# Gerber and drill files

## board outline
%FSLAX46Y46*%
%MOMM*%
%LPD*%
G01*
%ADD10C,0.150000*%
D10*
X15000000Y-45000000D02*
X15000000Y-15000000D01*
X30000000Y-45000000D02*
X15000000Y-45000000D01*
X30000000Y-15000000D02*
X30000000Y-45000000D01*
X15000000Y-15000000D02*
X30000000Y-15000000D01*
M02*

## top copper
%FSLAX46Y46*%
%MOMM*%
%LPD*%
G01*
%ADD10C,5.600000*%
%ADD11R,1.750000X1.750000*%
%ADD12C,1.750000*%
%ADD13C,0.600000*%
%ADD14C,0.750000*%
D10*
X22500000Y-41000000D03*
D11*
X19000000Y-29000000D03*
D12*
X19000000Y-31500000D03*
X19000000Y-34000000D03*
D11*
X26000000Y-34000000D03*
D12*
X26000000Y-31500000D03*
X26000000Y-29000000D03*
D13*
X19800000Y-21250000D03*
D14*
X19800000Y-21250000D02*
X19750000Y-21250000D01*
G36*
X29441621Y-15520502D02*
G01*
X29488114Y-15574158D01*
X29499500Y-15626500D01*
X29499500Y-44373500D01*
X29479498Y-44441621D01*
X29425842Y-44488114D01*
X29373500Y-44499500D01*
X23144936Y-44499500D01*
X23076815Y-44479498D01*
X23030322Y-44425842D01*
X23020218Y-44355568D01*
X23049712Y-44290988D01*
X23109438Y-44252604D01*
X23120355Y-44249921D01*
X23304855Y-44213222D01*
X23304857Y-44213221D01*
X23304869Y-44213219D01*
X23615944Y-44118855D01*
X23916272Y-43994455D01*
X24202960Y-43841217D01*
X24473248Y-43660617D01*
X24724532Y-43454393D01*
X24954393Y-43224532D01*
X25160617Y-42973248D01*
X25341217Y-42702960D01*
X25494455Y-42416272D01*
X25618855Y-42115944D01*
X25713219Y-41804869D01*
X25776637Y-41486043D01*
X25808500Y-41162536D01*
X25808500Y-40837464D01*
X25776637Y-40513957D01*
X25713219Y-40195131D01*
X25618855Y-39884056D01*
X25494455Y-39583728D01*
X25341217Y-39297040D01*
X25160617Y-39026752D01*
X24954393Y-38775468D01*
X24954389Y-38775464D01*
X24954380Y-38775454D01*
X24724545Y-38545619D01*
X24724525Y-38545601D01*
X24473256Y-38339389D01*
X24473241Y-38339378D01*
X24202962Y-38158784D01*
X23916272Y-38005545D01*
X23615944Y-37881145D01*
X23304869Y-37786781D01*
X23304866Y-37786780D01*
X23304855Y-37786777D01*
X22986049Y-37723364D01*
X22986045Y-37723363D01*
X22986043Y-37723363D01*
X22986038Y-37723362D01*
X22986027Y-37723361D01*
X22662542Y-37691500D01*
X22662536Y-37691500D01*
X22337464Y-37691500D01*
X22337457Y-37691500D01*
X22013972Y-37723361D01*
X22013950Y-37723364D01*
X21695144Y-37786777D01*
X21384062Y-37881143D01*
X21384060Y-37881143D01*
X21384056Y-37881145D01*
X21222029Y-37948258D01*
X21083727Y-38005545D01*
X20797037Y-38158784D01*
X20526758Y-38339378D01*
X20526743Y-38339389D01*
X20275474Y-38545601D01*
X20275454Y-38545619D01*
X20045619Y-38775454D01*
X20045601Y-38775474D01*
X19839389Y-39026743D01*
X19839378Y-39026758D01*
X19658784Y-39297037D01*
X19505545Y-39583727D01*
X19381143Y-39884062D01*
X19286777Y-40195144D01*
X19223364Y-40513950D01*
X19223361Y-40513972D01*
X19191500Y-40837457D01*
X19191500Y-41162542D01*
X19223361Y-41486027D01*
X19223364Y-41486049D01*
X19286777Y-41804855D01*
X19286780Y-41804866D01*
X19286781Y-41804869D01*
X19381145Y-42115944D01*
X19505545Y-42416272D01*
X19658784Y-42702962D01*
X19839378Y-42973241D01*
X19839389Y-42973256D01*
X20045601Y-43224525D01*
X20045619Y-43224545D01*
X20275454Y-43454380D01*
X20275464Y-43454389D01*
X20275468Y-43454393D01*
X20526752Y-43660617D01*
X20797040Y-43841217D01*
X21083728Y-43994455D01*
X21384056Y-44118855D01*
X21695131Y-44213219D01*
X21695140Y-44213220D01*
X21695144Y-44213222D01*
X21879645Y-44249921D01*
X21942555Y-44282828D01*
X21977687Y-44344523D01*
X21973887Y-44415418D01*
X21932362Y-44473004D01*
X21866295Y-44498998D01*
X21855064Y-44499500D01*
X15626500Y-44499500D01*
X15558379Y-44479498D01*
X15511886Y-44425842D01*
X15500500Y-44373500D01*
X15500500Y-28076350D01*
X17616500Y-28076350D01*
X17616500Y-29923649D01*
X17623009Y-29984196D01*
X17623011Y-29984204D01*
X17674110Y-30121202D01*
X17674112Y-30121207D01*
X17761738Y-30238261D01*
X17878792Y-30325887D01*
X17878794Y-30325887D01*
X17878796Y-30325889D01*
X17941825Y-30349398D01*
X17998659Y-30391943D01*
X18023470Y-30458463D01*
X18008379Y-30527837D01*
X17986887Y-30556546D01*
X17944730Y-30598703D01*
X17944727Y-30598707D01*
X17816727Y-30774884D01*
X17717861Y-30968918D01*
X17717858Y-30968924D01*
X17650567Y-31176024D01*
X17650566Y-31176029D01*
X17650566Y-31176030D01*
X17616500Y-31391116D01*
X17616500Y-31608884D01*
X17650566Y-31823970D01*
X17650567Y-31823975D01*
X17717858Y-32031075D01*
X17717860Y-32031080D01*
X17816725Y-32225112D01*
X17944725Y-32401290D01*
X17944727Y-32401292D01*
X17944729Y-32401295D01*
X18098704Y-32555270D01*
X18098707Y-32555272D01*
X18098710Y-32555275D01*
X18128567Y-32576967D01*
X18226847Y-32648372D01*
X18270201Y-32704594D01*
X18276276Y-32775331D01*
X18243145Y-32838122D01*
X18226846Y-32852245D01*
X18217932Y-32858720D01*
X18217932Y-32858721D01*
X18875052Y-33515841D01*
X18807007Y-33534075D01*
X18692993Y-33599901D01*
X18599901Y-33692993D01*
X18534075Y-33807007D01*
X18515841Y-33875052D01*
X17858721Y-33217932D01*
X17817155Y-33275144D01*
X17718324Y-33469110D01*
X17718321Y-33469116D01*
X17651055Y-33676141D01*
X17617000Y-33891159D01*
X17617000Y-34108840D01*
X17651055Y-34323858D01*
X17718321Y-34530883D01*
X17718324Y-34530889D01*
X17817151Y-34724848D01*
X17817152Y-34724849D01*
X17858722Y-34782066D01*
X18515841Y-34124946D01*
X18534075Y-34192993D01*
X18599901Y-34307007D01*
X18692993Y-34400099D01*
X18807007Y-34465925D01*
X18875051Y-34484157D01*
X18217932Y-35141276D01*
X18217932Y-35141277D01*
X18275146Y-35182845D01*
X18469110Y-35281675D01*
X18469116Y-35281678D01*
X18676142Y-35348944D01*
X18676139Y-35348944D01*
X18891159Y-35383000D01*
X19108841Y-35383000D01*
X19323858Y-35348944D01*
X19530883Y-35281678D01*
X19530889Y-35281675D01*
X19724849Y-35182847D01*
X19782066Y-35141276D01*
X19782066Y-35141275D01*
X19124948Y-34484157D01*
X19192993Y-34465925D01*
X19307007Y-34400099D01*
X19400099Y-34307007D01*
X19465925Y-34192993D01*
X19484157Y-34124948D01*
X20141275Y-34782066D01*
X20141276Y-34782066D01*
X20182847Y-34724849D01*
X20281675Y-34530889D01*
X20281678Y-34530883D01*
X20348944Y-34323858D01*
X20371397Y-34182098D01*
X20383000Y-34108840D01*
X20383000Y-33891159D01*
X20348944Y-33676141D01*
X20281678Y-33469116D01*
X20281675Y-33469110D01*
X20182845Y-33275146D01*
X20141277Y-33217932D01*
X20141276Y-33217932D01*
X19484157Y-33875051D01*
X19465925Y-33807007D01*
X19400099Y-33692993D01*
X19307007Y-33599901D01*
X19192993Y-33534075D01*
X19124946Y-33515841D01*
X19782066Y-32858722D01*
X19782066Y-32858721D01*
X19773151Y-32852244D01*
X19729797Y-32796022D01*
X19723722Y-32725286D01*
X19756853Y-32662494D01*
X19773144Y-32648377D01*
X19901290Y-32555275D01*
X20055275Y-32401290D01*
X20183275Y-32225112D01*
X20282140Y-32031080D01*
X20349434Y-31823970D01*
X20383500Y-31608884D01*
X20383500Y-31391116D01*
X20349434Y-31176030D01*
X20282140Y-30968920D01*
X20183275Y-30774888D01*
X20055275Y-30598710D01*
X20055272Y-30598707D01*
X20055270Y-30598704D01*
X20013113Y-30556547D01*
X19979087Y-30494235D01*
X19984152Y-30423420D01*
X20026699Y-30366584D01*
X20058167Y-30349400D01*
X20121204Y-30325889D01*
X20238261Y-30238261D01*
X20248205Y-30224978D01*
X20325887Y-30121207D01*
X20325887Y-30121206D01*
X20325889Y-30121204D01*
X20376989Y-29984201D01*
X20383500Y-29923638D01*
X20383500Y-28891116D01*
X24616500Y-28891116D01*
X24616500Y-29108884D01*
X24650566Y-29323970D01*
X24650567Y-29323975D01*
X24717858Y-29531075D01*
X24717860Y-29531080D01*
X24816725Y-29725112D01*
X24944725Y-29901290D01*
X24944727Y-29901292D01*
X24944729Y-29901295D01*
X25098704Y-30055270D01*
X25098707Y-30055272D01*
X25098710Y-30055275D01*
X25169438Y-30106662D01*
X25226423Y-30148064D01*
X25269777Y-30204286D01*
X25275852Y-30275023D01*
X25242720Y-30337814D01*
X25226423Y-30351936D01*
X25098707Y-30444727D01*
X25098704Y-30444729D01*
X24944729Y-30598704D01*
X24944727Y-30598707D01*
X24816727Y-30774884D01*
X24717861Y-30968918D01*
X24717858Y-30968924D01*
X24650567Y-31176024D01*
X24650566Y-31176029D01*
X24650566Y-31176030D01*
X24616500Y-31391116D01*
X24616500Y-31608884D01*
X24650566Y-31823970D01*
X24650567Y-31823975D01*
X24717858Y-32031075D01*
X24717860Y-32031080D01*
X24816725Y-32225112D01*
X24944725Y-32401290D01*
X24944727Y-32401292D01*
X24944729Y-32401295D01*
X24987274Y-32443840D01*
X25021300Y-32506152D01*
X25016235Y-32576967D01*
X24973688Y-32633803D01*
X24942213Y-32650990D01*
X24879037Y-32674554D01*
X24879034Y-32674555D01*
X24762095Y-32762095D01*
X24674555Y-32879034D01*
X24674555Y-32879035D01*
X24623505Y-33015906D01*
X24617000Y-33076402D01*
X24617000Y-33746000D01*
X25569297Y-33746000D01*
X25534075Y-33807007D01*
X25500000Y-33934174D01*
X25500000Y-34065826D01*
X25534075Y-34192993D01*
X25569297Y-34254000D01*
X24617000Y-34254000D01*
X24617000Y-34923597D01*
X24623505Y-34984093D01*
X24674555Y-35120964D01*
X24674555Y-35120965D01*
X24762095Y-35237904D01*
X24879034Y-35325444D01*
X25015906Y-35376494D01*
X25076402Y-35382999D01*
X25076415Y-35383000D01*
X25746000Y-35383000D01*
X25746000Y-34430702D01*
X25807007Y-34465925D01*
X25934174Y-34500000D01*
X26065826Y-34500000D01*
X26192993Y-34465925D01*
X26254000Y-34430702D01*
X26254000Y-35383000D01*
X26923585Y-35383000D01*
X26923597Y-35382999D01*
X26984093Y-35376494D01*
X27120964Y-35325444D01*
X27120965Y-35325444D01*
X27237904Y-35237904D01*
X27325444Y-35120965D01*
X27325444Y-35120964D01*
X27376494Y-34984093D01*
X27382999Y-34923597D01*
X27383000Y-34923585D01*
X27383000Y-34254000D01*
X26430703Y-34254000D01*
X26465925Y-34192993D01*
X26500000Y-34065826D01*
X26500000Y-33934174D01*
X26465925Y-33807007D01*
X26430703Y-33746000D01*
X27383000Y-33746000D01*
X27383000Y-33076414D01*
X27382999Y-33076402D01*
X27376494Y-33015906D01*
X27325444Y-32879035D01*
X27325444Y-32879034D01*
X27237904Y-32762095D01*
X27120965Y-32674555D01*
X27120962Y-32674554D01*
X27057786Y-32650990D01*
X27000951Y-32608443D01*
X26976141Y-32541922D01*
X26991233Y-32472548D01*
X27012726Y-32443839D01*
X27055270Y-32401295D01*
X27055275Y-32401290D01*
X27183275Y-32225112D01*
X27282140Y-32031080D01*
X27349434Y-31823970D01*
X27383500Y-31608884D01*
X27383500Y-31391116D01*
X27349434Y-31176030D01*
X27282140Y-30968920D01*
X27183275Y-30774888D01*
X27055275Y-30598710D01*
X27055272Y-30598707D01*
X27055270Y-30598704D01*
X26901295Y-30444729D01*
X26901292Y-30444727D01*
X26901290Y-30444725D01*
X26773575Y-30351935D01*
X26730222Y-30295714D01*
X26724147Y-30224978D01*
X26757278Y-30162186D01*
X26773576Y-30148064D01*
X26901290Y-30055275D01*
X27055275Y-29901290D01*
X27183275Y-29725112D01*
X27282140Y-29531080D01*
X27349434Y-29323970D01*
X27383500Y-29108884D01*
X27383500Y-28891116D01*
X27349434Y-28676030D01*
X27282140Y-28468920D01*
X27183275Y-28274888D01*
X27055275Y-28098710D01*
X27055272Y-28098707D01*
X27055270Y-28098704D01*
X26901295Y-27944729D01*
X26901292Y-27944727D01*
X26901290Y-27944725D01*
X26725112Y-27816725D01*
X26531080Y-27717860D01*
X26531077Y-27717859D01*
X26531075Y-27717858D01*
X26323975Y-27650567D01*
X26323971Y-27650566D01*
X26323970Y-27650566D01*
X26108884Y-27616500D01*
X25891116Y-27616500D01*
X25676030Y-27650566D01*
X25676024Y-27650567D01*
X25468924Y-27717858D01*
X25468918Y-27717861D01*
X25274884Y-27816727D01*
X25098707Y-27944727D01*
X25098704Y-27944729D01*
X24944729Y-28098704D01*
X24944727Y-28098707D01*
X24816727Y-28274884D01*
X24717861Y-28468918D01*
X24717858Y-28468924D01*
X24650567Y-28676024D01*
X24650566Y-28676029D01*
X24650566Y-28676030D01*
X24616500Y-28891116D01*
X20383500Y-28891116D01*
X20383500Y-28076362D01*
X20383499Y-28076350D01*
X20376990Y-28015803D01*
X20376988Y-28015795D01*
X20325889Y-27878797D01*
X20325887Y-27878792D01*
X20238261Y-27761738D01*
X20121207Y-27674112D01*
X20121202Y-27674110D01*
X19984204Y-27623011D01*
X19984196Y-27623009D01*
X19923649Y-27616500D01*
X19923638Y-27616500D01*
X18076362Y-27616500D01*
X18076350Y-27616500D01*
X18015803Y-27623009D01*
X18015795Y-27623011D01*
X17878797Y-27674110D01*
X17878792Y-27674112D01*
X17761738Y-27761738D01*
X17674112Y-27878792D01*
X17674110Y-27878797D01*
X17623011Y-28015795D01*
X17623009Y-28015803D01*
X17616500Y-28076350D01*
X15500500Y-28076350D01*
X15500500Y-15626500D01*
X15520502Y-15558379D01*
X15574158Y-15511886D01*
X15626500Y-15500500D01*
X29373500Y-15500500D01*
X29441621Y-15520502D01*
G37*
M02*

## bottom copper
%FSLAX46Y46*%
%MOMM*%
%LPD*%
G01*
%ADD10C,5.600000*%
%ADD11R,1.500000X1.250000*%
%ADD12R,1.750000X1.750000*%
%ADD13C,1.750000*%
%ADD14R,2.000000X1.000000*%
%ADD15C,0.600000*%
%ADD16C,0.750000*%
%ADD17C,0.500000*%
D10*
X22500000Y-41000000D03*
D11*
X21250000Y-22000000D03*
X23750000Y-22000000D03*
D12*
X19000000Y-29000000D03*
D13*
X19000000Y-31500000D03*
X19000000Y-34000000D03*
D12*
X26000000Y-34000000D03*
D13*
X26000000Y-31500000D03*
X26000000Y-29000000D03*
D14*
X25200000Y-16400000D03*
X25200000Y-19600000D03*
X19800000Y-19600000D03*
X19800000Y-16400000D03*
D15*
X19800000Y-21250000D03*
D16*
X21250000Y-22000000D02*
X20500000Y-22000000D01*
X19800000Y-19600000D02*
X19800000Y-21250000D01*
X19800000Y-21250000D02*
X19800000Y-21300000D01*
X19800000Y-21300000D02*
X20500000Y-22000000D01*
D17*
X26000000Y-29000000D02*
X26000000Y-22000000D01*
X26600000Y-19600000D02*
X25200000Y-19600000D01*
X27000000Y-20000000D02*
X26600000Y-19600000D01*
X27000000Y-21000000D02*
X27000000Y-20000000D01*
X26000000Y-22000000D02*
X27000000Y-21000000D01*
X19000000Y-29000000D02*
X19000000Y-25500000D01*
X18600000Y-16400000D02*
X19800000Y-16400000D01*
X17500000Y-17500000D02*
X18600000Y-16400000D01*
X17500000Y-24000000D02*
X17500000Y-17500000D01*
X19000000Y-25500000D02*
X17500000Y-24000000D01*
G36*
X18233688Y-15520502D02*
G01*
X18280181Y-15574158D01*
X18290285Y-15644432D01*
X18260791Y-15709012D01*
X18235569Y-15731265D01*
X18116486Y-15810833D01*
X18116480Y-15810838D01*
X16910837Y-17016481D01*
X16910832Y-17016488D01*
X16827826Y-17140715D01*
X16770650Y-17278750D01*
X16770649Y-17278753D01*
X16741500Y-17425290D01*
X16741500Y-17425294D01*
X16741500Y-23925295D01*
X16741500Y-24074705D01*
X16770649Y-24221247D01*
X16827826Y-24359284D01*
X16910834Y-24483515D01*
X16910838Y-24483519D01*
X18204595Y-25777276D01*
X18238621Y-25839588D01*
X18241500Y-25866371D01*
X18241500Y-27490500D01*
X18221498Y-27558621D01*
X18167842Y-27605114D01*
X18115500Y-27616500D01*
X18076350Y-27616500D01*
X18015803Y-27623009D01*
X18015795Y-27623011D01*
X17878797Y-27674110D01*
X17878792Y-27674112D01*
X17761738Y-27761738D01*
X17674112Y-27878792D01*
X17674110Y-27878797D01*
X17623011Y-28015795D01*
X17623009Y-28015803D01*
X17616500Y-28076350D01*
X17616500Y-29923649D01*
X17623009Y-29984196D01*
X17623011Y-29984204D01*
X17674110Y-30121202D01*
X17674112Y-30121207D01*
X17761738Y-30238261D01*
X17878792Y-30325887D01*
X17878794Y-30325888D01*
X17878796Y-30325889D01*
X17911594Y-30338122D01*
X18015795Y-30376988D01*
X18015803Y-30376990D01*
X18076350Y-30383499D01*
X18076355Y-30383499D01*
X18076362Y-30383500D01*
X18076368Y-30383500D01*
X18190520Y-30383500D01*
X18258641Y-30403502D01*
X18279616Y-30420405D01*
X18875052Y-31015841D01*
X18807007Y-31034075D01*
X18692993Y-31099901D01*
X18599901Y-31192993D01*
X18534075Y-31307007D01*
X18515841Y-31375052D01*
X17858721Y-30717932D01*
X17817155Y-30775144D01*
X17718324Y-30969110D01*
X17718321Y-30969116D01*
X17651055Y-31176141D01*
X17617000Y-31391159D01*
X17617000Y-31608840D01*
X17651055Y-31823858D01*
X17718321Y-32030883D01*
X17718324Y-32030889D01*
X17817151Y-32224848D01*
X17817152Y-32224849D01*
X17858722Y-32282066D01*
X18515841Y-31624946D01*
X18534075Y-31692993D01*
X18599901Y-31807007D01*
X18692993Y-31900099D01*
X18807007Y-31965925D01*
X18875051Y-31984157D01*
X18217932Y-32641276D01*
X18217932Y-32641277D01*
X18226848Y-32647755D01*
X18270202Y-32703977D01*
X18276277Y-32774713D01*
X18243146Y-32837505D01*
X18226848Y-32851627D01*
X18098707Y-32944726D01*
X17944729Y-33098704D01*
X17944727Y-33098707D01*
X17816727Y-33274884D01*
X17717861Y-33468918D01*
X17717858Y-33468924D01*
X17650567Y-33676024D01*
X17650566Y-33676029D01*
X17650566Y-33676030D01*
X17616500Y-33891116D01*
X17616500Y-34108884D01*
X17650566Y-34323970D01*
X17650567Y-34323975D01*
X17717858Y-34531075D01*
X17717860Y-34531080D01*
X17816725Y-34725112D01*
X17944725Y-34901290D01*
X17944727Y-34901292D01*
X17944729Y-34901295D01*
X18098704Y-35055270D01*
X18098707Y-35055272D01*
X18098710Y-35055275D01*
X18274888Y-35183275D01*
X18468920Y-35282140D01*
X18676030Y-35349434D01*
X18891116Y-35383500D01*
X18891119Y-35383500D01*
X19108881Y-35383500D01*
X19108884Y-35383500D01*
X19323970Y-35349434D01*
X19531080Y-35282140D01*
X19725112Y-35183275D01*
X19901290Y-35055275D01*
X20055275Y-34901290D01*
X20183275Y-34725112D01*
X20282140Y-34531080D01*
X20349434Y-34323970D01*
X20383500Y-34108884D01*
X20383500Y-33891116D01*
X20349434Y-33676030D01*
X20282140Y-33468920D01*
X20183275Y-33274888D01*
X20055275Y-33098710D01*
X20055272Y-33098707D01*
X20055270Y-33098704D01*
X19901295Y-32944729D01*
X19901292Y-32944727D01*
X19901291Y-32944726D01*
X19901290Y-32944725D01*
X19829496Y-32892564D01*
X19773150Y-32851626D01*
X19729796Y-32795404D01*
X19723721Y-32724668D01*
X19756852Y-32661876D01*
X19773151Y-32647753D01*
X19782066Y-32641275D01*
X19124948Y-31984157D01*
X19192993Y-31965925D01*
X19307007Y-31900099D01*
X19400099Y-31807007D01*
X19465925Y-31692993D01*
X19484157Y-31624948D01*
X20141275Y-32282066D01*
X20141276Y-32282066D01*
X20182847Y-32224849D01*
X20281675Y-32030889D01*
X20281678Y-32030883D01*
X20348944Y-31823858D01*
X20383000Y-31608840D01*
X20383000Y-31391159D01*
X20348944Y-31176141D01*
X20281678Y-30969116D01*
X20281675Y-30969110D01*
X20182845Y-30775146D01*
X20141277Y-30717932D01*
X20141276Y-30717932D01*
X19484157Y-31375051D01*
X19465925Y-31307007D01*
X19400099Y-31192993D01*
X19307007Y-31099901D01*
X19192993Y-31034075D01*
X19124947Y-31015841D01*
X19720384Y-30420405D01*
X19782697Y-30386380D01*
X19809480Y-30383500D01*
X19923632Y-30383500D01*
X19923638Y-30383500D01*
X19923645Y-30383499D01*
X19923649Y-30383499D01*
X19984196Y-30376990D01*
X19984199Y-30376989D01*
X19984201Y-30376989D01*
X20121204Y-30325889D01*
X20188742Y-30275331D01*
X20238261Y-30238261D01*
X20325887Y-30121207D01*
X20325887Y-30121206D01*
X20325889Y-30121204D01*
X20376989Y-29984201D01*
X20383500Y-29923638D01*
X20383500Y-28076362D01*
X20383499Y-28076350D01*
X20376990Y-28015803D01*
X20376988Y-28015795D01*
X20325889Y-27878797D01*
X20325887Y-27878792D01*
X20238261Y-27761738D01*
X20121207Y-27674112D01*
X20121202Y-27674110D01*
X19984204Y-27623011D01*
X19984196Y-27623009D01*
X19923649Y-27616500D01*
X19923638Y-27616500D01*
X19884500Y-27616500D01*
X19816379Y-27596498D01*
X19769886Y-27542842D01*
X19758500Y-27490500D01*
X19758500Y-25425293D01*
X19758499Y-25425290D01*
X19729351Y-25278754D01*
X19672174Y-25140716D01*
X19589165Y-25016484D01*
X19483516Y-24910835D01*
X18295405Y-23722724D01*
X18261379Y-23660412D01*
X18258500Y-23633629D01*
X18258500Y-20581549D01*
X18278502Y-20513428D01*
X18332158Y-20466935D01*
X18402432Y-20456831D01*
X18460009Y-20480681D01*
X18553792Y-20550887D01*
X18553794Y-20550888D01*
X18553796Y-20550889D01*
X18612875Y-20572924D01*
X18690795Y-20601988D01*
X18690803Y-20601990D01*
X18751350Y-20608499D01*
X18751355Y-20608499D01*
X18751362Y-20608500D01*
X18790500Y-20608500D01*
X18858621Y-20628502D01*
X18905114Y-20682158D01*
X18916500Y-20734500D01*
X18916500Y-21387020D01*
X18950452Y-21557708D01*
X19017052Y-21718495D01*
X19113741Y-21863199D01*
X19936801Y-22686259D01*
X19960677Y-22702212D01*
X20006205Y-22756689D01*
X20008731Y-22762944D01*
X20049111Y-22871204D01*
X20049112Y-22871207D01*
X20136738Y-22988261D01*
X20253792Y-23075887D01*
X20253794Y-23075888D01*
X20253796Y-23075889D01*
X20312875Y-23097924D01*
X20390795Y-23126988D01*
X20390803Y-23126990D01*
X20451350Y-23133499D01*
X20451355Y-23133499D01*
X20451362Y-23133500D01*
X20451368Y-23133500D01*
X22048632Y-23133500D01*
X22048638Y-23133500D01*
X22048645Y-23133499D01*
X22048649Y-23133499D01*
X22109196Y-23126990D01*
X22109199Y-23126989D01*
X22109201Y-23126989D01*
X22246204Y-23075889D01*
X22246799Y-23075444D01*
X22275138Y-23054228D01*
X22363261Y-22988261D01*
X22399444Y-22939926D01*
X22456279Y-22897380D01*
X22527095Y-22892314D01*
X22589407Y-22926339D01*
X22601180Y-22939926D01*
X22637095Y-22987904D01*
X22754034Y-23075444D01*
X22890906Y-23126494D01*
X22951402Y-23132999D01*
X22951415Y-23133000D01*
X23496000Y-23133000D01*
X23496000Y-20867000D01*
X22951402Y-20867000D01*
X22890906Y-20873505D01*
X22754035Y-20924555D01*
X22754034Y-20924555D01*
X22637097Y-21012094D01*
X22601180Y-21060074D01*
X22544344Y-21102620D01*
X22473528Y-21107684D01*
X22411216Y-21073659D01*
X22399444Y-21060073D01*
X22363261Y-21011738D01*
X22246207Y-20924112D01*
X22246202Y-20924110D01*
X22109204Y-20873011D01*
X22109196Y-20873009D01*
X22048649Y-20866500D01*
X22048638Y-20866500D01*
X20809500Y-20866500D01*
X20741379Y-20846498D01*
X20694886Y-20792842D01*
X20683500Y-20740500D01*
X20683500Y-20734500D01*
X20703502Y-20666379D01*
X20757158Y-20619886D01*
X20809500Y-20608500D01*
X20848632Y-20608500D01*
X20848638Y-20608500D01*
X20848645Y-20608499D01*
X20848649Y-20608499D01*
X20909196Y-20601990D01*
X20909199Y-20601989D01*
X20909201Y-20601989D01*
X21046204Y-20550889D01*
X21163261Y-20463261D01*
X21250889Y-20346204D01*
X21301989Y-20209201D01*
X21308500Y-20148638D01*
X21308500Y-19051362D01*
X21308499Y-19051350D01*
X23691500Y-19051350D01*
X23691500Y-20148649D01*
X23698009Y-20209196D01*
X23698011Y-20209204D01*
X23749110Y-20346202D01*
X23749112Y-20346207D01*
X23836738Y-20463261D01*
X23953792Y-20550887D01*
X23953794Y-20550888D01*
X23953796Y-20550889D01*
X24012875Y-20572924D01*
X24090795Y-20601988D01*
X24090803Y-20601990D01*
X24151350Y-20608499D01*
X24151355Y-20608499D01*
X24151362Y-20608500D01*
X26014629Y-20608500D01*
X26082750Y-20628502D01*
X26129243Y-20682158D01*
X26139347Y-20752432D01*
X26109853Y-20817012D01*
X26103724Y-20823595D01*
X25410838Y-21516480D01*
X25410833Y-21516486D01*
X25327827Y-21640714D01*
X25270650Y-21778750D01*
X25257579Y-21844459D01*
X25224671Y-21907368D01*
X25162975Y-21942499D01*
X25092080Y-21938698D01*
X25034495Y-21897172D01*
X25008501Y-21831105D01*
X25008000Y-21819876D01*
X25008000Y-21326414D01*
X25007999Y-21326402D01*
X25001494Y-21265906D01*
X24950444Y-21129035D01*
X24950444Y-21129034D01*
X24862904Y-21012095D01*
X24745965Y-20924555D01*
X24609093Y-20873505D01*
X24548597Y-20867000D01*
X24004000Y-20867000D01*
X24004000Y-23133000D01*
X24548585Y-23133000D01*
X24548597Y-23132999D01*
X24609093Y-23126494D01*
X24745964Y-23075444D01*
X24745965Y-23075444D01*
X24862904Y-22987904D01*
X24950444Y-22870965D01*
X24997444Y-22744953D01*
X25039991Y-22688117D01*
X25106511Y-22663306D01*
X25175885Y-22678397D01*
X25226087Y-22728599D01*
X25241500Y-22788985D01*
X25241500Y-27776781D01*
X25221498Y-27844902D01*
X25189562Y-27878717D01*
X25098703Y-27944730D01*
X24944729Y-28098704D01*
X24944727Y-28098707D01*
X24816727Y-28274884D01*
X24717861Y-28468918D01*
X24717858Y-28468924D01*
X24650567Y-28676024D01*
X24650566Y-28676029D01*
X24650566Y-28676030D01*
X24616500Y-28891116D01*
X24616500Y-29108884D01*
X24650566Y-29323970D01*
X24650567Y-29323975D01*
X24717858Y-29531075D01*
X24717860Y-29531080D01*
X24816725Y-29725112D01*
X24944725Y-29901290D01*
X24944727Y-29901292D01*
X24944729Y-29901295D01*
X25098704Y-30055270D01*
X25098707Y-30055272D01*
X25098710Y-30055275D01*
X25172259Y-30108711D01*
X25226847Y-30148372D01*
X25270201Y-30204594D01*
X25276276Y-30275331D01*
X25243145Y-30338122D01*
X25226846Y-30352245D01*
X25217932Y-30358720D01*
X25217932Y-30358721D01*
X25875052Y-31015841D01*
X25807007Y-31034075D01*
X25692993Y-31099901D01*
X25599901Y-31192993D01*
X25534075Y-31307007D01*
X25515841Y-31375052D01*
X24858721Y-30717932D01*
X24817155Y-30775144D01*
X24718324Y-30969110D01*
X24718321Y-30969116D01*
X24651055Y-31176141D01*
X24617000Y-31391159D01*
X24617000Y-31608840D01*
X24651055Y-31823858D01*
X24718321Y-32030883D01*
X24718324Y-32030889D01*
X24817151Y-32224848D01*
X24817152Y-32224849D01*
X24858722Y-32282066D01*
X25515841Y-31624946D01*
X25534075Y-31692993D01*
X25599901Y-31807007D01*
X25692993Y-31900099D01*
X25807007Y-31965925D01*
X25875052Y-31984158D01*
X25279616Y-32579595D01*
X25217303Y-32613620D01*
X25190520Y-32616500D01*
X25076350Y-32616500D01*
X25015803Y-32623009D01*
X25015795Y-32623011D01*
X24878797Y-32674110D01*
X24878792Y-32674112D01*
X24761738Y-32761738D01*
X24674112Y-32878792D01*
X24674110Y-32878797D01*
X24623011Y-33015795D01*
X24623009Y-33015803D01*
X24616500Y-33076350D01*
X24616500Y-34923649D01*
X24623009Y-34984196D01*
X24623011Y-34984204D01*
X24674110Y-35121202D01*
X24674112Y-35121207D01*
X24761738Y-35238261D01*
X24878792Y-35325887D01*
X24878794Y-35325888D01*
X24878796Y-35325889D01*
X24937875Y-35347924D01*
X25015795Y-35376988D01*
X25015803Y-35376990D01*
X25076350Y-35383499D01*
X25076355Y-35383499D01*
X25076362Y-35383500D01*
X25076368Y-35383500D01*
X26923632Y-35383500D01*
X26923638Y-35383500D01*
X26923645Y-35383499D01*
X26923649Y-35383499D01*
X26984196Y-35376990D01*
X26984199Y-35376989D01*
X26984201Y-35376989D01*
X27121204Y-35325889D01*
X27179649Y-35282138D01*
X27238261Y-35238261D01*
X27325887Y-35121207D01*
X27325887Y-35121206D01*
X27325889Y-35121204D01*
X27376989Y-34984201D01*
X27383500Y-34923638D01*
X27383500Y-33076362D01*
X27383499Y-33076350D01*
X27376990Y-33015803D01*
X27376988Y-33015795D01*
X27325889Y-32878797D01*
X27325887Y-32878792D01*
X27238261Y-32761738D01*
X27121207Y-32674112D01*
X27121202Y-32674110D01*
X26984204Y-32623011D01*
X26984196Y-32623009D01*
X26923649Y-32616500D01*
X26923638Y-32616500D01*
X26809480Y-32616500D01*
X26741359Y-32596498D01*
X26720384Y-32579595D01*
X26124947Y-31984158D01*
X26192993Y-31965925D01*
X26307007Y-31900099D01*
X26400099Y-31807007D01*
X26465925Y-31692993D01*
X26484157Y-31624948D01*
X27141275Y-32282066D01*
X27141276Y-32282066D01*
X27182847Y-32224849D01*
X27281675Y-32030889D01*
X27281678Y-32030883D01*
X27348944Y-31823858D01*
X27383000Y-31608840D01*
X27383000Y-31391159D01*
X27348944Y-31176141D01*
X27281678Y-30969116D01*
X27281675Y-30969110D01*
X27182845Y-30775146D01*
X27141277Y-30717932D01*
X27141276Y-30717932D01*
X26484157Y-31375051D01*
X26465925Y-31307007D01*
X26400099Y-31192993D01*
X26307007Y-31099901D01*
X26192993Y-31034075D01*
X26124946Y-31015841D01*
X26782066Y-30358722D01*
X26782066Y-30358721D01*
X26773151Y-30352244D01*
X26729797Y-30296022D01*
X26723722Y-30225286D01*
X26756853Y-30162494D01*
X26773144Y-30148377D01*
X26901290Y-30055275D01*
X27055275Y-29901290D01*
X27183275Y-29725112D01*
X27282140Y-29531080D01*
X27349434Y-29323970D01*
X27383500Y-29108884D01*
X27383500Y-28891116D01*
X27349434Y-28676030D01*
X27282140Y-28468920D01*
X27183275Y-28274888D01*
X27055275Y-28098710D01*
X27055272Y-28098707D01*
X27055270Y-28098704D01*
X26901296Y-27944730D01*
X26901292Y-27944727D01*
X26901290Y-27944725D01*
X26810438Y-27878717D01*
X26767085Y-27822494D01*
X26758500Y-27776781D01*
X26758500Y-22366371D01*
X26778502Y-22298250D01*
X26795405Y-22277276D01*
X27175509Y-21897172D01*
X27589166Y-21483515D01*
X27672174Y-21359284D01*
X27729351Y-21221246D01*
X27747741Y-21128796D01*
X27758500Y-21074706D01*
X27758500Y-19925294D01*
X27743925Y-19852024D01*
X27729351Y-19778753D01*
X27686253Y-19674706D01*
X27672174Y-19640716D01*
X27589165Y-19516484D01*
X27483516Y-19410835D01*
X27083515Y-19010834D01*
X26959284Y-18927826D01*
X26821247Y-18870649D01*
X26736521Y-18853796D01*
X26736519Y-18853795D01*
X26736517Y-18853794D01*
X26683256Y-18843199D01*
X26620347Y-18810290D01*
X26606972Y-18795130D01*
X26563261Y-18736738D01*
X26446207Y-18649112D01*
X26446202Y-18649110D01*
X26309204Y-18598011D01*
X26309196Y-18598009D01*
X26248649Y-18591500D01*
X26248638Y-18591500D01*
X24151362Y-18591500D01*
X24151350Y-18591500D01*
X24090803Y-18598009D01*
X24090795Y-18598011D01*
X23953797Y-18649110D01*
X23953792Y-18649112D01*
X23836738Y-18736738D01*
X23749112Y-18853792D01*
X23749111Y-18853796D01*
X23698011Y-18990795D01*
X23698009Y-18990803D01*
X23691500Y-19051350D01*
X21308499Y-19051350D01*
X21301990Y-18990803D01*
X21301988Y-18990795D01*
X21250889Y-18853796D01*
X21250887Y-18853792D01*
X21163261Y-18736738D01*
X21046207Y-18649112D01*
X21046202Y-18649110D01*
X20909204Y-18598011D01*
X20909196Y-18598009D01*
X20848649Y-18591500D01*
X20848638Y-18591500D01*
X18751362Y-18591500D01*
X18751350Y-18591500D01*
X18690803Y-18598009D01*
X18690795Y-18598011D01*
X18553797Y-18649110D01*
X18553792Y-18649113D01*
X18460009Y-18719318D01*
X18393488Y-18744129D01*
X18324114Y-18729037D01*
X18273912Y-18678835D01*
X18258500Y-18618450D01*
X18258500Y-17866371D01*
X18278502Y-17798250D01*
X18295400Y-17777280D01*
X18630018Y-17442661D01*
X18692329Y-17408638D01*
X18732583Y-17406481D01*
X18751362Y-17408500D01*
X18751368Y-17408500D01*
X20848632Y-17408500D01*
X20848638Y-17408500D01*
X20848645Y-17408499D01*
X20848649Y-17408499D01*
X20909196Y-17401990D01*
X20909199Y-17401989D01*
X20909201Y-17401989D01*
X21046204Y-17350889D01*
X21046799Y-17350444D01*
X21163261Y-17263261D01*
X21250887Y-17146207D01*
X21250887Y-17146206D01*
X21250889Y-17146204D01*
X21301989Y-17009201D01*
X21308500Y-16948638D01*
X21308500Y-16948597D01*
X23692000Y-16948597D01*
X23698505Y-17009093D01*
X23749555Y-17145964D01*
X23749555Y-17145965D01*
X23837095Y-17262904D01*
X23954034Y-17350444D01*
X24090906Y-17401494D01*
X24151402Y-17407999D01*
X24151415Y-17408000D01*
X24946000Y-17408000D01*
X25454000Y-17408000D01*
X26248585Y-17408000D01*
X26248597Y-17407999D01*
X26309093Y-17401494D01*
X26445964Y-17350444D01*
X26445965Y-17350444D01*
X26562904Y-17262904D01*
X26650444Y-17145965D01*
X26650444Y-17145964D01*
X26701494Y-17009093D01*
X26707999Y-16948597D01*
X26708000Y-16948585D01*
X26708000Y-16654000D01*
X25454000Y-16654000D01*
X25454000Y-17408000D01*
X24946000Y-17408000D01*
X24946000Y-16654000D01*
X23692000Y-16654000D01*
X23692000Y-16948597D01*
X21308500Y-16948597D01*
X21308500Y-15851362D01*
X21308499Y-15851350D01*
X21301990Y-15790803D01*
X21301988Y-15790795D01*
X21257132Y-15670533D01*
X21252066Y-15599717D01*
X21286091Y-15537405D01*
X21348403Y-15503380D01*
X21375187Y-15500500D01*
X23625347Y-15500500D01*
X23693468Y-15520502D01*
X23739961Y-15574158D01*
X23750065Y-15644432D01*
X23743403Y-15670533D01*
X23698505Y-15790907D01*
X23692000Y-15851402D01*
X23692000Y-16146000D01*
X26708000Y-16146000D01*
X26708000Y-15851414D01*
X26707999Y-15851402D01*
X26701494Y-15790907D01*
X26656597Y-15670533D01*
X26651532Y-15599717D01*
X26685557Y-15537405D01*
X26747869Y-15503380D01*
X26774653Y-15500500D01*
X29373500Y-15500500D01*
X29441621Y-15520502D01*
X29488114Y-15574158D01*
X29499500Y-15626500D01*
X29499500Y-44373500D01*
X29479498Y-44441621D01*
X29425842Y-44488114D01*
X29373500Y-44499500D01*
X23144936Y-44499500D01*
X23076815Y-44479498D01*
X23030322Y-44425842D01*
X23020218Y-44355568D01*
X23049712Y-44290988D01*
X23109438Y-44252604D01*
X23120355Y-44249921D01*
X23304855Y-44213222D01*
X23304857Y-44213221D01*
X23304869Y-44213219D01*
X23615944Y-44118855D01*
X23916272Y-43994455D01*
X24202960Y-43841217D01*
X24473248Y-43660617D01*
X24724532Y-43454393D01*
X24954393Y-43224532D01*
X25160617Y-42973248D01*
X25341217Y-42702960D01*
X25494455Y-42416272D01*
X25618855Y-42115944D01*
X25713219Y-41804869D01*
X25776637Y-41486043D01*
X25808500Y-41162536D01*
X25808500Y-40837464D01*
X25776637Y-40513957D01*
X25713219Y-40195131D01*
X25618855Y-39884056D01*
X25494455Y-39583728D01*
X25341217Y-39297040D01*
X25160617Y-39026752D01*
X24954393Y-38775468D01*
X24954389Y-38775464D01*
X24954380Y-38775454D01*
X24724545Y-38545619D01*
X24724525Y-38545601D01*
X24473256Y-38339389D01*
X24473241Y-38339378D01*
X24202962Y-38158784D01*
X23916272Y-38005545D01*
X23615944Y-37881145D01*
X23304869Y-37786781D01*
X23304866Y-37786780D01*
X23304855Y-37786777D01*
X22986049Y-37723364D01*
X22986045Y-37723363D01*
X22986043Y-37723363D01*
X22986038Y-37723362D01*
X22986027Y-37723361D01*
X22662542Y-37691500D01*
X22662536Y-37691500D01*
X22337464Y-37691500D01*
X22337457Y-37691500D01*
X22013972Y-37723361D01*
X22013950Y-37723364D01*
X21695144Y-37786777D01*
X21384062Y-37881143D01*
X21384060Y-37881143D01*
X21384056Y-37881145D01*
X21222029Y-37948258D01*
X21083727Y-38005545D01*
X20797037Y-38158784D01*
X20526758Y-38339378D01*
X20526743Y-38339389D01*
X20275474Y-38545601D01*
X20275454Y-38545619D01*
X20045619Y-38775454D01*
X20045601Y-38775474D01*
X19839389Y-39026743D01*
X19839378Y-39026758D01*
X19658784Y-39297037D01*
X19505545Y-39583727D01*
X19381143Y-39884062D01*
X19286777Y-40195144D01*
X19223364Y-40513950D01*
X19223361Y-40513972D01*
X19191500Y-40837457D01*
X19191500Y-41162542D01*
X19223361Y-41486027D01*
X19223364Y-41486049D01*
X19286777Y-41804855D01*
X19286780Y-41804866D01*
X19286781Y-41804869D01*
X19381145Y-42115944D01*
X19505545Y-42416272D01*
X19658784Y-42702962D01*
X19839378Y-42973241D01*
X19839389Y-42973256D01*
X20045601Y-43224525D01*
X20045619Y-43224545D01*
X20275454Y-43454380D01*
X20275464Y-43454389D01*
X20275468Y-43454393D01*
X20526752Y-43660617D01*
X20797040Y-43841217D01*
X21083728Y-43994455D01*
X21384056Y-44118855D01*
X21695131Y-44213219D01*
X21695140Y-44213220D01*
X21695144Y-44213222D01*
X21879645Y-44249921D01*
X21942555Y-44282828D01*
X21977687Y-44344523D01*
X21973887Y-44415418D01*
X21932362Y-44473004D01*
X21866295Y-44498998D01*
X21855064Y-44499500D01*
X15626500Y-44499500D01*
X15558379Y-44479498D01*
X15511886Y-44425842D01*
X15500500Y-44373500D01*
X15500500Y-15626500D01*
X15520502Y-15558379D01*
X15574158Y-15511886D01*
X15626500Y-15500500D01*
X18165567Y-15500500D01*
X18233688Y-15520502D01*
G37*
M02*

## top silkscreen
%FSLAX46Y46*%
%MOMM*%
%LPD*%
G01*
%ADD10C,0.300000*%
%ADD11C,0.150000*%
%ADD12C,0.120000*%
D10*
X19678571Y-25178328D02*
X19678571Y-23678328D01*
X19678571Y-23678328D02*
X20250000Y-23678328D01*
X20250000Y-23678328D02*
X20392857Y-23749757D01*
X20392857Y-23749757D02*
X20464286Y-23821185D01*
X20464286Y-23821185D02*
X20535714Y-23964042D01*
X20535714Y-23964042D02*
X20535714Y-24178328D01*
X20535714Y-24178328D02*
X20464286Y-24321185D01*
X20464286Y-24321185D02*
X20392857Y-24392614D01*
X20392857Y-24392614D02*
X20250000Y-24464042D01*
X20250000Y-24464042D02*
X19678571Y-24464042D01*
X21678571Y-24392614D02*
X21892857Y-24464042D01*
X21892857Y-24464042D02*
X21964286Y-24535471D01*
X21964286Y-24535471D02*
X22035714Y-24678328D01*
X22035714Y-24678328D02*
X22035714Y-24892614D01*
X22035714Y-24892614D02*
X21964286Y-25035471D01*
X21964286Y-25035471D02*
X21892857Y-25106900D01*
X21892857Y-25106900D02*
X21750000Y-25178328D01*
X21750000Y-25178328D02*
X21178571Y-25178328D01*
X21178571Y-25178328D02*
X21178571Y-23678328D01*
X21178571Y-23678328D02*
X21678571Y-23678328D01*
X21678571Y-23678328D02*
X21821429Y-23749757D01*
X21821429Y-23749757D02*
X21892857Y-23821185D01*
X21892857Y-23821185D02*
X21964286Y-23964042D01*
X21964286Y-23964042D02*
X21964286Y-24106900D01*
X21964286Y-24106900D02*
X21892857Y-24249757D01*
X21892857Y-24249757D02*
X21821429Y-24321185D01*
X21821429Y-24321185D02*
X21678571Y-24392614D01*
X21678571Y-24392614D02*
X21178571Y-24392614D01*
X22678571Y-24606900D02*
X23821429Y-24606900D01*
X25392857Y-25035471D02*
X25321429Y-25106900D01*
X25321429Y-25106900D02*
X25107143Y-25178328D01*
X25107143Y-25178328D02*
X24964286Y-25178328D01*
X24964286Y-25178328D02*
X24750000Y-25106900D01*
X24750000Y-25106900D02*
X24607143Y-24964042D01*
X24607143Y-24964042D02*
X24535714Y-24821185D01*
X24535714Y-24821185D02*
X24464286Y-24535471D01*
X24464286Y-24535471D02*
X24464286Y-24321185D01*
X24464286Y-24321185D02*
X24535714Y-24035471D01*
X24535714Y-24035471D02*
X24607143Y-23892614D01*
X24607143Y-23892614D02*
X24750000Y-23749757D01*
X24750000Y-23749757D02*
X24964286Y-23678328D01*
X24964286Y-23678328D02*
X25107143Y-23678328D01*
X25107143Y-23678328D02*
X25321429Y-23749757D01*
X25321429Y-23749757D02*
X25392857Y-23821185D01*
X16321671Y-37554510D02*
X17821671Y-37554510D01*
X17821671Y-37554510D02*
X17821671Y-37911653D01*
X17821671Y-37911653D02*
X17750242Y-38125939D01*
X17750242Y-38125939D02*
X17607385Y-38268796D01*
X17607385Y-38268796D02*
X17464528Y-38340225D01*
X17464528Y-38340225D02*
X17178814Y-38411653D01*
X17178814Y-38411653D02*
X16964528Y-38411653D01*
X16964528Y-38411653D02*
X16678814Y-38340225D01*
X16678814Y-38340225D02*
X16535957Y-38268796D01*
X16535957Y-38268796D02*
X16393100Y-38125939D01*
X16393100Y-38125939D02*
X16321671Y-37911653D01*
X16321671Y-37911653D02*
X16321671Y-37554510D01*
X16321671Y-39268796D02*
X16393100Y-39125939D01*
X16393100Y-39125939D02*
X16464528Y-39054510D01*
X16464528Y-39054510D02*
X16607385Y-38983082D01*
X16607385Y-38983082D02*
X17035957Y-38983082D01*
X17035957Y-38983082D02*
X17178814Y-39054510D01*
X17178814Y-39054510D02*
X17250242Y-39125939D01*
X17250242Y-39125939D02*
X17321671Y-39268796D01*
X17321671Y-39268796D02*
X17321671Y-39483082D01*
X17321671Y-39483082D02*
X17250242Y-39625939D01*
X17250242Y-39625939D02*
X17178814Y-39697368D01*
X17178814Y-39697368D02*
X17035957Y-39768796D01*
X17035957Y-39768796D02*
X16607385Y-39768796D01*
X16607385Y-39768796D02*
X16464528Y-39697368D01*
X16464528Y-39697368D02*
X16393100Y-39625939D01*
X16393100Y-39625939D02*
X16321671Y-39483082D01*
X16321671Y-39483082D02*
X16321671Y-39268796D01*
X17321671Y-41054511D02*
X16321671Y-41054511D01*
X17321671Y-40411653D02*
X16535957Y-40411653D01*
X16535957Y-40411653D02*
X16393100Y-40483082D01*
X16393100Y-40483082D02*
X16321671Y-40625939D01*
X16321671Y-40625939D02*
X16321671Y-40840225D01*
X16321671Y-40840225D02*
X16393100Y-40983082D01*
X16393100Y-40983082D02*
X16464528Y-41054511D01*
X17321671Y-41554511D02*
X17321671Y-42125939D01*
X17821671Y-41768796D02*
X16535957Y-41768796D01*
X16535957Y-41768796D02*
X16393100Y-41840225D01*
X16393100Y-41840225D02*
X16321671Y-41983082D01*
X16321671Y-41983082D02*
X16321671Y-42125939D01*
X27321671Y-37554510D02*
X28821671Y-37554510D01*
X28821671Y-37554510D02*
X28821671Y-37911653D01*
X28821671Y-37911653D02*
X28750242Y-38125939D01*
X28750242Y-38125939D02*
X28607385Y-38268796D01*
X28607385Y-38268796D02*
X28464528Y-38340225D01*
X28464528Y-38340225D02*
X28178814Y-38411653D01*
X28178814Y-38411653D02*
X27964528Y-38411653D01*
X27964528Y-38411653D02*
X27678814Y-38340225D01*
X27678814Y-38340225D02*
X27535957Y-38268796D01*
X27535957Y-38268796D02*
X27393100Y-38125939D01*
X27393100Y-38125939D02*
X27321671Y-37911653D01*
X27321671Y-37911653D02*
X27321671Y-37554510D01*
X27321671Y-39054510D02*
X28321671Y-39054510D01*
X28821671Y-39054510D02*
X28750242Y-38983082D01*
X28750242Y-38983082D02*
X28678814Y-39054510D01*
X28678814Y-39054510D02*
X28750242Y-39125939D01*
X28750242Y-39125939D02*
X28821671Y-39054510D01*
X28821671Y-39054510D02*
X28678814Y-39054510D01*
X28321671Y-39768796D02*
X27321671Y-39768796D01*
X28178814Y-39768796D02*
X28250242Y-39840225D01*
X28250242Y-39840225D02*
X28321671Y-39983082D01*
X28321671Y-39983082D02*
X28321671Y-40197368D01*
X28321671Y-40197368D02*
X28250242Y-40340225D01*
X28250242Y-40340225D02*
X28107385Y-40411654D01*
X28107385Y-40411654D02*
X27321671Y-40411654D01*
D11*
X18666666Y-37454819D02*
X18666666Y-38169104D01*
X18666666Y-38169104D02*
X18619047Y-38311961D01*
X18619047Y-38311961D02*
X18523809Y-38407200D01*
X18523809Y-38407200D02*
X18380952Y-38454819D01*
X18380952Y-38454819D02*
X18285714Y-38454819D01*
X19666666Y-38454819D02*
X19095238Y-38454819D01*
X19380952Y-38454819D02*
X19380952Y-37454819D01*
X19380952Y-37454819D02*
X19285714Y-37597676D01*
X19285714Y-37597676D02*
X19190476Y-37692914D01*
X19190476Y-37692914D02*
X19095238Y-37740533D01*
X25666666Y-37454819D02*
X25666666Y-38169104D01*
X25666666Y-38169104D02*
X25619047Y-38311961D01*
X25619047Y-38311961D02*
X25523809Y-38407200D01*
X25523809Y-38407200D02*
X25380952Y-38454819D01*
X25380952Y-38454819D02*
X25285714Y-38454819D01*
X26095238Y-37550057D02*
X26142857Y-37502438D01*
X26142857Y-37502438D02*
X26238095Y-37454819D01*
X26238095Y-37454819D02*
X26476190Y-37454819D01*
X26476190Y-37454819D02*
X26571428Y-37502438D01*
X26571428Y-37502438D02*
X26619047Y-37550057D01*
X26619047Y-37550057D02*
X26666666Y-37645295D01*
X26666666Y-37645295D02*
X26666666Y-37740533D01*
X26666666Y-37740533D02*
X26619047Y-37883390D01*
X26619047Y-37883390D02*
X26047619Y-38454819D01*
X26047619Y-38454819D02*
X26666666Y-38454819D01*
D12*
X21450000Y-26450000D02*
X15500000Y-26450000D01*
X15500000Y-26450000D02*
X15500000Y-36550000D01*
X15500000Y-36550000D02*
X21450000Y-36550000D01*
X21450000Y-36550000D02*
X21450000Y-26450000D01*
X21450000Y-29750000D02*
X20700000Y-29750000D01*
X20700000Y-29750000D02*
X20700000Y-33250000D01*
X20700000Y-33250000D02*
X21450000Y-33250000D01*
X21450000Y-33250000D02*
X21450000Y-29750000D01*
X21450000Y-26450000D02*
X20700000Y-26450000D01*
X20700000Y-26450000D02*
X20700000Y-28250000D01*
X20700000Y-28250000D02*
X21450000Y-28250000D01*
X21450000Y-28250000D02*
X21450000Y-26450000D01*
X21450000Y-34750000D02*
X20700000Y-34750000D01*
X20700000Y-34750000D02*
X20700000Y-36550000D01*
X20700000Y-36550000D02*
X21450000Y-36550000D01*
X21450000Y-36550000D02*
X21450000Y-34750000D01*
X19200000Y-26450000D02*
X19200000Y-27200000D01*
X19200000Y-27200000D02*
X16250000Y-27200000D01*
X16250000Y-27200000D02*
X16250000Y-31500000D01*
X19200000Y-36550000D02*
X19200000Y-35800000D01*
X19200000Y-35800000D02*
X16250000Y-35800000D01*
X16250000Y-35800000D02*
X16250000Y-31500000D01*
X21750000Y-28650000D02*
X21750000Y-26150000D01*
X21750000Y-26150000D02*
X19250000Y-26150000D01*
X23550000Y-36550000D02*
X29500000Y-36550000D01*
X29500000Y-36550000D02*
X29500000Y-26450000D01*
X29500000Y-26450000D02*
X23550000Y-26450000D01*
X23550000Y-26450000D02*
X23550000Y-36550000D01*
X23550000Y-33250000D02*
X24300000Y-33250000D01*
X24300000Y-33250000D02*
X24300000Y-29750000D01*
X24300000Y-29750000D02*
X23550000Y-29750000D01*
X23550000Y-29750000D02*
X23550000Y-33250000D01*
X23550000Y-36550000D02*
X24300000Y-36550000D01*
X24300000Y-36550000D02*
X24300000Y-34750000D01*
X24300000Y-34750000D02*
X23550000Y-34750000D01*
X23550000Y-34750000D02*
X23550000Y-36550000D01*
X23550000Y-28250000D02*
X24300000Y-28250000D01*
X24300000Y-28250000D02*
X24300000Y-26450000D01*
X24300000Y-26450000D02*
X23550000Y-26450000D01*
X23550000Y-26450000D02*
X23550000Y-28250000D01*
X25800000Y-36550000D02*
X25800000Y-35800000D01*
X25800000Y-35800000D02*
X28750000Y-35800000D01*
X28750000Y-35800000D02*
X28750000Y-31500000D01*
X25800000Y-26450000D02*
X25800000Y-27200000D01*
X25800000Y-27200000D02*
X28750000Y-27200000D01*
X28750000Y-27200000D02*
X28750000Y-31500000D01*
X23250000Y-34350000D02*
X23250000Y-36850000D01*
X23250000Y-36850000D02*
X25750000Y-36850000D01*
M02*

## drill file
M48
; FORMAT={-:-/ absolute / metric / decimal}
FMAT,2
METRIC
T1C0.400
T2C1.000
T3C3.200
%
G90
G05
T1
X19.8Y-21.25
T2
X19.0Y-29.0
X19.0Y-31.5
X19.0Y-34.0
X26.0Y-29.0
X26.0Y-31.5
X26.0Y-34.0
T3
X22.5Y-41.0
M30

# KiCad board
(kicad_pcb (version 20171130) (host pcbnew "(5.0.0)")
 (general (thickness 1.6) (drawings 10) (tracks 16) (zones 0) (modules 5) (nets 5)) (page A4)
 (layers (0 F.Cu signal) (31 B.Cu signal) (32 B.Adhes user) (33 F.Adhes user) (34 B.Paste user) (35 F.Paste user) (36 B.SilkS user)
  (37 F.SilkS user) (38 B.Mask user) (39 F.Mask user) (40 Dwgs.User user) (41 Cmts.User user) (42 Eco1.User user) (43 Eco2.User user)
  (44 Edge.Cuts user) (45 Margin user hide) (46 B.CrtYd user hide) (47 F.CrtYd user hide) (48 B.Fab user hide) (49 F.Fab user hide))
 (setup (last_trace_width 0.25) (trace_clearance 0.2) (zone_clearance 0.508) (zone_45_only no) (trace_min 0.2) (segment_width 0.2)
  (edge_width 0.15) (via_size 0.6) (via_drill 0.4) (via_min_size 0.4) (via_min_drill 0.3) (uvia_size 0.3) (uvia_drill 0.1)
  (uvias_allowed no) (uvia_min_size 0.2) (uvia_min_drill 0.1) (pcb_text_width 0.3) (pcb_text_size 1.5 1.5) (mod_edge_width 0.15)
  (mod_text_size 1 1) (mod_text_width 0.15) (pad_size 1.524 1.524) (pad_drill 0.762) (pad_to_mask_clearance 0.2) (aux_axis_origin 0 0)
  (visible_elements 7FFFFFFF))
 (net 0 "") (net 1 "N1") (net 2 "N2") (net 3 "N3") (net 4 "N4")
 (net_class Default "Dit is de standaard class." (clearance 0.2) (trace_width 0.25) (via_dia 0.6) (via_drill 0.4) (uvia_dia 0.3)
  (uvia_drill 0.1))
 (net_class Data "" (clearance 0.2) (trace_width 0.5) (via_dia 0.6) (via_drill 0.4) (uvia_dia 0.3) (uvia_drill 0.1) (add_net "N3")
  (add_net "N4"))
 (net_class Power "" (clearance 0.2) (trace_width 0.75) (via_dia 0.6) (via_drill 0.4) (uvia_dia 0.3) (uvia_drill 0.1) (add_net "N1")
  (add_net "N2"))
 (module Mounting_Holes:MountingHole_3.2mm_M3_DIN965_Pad (layer F.Cu) (at 22.5 41)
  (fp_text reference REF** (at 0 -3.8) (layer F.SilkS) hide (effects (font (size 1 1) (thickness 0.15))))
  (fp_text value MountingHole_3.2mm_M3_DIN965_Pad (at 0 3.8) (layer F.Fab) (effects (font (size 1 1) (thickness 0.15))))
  (pad 1 thru_hole circle (at 0 0) (size 5.6 5.6) (drill 3.2) (layers *.Cu *.Mask)))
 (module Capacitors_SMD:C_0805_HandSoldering (layer B.Cu) (at 22.5 22)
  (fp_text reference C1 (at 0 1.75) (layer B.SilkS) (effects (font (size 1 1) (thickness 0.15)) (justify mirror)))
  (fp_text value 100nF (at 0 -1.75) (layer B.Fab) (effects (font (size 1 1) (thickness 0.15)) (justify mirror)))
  (pad 1 smd rect (at -1.25 0) (size 1.5 1.25) (layers B.Cu B.Paste B.Mask) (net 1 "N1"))
  (pad 2 smd rect (at 1.25 0) (size 1.5 1.25) (layers B.Cu B.Paste B.Mask) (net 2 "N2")))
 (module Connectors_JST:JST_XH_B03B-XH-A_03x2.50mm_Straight (layer F.Cu) (at 19 29 270)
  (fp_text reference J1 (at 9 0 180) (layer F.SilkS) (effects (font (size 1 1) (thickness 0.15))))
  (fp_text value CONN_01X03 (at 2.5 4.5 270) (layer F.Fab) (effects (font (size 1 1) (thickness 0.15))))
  (fp_line (start -2.55 -2.45) (end -2.55 3.5) (layer F.SilkS) (width 0.12))
  (fp_line (start -2.55 3.5) (end 7.55 3.5) (layer F.SilkS) (width 0.12))
  (fp_line (start 7.55 3.5) (end 7.55 -2.45) (layer F.SilkS) (width 0.12))
  (fp_line (start 7.55 -2.45) (end -2.55 -2.45) (layer F.SilkS) (width 0.12))
  (fp_line (start 0.75 -2.45) (end 0.75 -1.7) (layer F.SilkS) (width 0.12))
  (fp_line (start 0.75 -1.7) (end 4.25 -1.7) (layer F.SilkS) (width 0.12))
  (fp_line (start 4.25 -1.7) (end 4.25 -2.45) (layer F.SilkS) (width 0.12))
  (fp_line (start 4.25 -2.45) (end 0.75 -2.45) (layer F.SilkS) (width 0.12))
  (fp_line (start -2.55 -2.45) (end -2.55 -1.7) (layer F.SilkS) (width 0.12))
  (fp_line (start -2.55 -1.7) (end -0.75 -1.7) (layer F.SilkS) (width 0.12))
  (fp_line (start -0.75 -1.7) (end -0.75 -2.45) (layer F.SilkS) (width 0.12))
  (fp_line (start -0.75 -2.45) (end -2.55 -2.45) (layer F.SilkS) (width 0.12))
  (fp_line (start 5.75 -2.45) (end 5.75 -1.7) (layer F.SilkS) (width 0.12))
  (fp_line (start 5.75 -1.7) (end 7.55 -1.7) (layer F.SilkS) (width 0.12))
  (fp_line (start 7.55 -1.7) (end 7.55 -2.45) (layer F.SilkS) (width 0.12))
  (fp_line (start 7.55 -2.45) (end 5.75 -2.45) (layer F.SilkS) (width 0.12))
  (fp_line (start -2.55 -0.2) (end -1.8 -0.2) (layer F.SilkS) (width 0.12))
  (fp_line (start -1.8 -0.2) (end -1.8 2.75) (layer F.SilkS) (width 0.12))
  (fp_line (start -1.8 2.75) (end 2.5 2.75) (layer F.SilkS) (width 0.12))
  (fp_line (start 7.55 -0.2) (end 6.8 -0.2) (layer F.SilkS) (width 0.12))
  (fp_line (start 6.8 -0.2) (end 6.8 2.75) (layer F.SilkS) (width 0.12))
  (fp_line (start 6.8 2.75) (end 2.5 2.75) (layer F.SilkS) (width 0.12))
  (fp_line (start -0.35 -2.75) (end -2.85 -2.75) (layer F.SilkS) (width 0.12))
  (fp_line (start -2.85 -2.75) (end -2.85 -0.25) (layer F.SilkS) (width 0.12))
  (pad 1 thru_hole rect (at 0 0 270) (size 1.75 1.75) (drill 1) (layers *.Cu *.Mask) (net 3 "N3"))
  (pad 2 thru_hole circle (at 2.5 0 270) (size 1.75 1.75) (drill 1) (layers *.Cu *.Mask) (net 2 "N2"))
  (pad 3 thru_hole circle (at 5 0 270) (size 1.75 1.75) (drill 1) (layers *.Cu *.Mask) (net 1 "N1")))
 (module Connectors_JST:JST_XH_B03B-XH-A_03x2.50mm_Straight (layer F.Cu) (at 26 34 90)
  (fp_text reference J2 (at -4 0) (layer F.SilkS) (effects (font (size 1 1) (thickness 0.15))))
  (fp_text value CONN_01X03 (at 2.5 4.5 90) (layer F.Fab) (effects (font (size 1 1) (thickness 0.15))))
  (fp_line (start -2.55 -2.45) (end -2.55 3.5) (layer F.SilkS) (width 0.12))
  (fp_line (start -2.55 3.5) (end 7.55 3.5) (layer F.SilkS) (width 0.12))
  (fp_line (start 7.55 3.5) (end 7.55 -2.45) (layer F.SilkS) (width 0.12))
  (fp_line (start 7.55 -2.45) (end -2.55 -2.45) (layer F.SilkS) (width 0.12))
  (fp_line (start 0.75 -2.45) (end 0.75 -1.7) (layer F.SilkS) (width 0.12))
  (fp_line (start 0.75 -1.7) (end 4.25 -1.7) (layer F.SilkS) (width 0.12))
  (fp_line (start 4.25 -1.7) (end 4.25 -2.45) (layer F.SilkS) (width 0.12))
  (fp_line (start 4.25 -2.45) (end 0.75 -2.45) (layer F.SilkS) (width 0.12))
  (fp_line (start -2.55 -2.45) (end -2.55 -1.7) (layer F.SilkS) (width 0.12))
  (fp_line (start -2.55 -1.7) (end -0.75 -1.7) (layer F.SilkS) (width 0.12))
  (fp_line (start -0.75 -1.7) (end -0.75 -2.45) (layer F.SilkS) (width 0.12))
  (fp_line (start -0.75 -2.45) (end -2.55 -2.45) (layer F.SilkS) (width 0.12))
  (fp_line (start 5.75 -2.45) (end 5.75 -1.7) (layer F.SilkS) (width 0.12))
  (fp_line (start 5.75 -1.7) (end 7.55 -1.7) (layer F.SilkS) (width 0.12))
  (fp_line (start 7.55 -1.7) (end 7.55 -2.45) (layer F.SilkS) (width 0.12))
  (fp_line (start 7.55 -2.45) (end 5.75 -2.45) (layer F.SilkS) (width 0.12))
  (fp_line (start -2.55 -0.2) (end -1.8 -0.2) (layer F.SilkS) (width 0.12))
  (fp_line (start -1.8 -0.2) (end -1.8 2.75) (layer F.SilkS) (width 0.12))
  (fp_line (start -1.8 2.75) (end 2.5 2.75) (layer F.SilkS) (width 0.12))
  (fp_line (start 7.55 -0.2) (end 6.8 -0.2) (layer F.SilkS) (width 0.12))
  (fp_line (start 6.8 -0.2) (end 6.8 2.75) (layer F.SilkS) (width 0.12))
  (fp_line (start 6.8 2.75) (end 2.5 2.75) (layer F.SilkS) (width 0.12))
  (fp_line (start -0.35 -2.75) (end -2.85 -2.75) (layer F.SilkS) (width 0.12))
  (fp_line (start -2.85 -2.75) (end -2.85 -0.25) (layer F.SilkS) (width 0.12))
  (pad 1 thru_hole rect (at 0 0 90) (size 1.75 1.75) (drill 1) (layers *.Cu *.Mask) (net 1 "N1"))
  (pad 2 thru_hole circle (at 2.5 0 90) (size 1.75 1.75) (drill 1) (layers *.Cu *.Mask) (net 2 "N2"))
  (pad 3 thru_hole circle (at 5 0 90) (size 1.75 1.75) (drill 1) (layers *.Cu *.Mask) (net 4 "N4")))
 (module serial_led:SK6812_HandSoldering (layer B.Cu) (at 22.5 18)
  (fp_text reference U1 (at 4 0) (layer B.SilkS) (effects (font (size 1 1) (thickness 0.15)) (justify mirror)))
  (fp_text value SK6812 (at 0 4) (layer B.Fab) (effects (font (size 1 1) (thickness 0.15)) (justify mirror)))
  (pad 1 smd rect (at 2.7 -1.6) (size 2 1) (layers B.Cu B.Paste B.Mask) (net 2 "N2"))
  (pad 2 smd rect (at 2.7 1.6) (size 2 1) (layers B.Cu B.Paste B.Mask) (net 4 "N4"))
  (pad 3 smd rect (at -2.7 1.6) (size 2 1) (layers B.Cu B.Paste B.Mask) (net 1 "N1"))
  (pad 4 smd rect (at -2.7 -1.6) (size 2 1) (layers B.Cu B.Paste B.Mask) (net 3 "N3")))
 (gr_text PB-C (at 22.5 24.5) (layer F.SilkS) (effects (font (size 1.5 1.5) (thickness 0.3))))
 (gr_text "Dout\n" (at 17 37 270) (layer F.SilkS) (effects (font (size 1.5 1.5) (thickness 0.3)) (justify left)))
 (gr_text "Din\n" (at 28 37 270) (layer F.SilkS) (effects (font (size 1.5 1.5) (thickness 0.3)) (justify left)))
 (gr_line (start 15 45) (end 15 15) (angle 90) (layer Edge.Cuts) (width 0.15))
 (gr_line (start 30 45) (end 15 45) (angle 90) (layer Edge.Cuts) (width 0.15))
 (gr_line (start 30 15) (end 30 45) (angle 90) (layer Edge.Cuts) (width 0.15))
 (gr_line (start 15 15) (end 30 15) (angle 90) (layer Edge.Cuts) (width 0.15))
 (via (at 19.8 21.25) (size 0.6) (drill 0.4) (layers F.Cu B.Cu) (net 1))
 (segment (start 19.8 21.25) (end 19.75 21.25) (width 0.75) (layer F.Cu) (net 1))
 (segment (start 21.25 22) (end 20.5 22) (width 0.75) (layer B.Cu) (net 1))
 (segment (start 19.8 19.6) (end 19.8 21.25) (width 0.75) (layer B.Cu) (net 1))
 (segment (start 19.8 21.25) (end 19.8 21.3) (width 0.75) (layer B.Cu) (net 1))
 (segment (start 19.8 21.3) (end 20.5 22) (width 0.75) (layer B.Cu) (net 1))
 (segment (start 26 29) (end 26 22) (width 0.5) (layer B.Cu) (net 4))
 (segment (start 26.6 19.6) (end 25.2 19.6) (width 0.5) (layer B.Cu) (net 4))
 (segment (start 27 20) (end 26.6 19.6) (width 0.5) (layer B.Cu) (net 4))
 (segment (start 27 21) (end 27 20) (width 0.5) (layer B.Cu) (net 4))
 (segment (start 26 22) (end 27 21) (width 0.5) (layer B.Cu) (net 4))
 (segment (start 19 29) (end 19 25.5) (width 0.5) (layer B.Cu) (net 3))
 (segment (start 18.6 16.4) (end 19.8 16.4) (width 0.5) (layer B.Cu) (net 3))
 (segment (start 17.5 17.5) (end 18.6 16.4) (width 0.5) (layer B.Cu) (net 3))
 (segment (start 17.5 24) (end 17.5 17.5) (width 0.5) (layer B.Cu) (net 3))
 (segment (start 19 25.5) (end 17.5 24) (width 0.5) (layer B.Cu) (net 3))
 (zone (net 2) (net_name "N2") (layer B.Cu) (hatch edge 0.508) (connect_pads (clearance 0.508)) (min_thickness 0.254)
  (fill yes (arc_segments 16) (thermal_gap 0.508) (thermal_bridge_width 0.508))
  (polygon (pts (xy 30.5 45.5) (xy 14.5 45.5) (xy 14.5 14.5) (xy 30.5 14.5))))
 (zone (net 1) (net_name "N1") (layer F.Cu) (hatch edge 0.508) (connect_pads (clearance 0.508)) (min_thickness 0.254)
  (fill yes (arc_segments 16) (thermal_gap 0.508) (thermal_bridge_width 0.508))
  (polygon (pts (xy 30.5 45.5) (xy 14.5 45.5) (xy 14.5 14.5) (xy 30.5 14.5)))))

